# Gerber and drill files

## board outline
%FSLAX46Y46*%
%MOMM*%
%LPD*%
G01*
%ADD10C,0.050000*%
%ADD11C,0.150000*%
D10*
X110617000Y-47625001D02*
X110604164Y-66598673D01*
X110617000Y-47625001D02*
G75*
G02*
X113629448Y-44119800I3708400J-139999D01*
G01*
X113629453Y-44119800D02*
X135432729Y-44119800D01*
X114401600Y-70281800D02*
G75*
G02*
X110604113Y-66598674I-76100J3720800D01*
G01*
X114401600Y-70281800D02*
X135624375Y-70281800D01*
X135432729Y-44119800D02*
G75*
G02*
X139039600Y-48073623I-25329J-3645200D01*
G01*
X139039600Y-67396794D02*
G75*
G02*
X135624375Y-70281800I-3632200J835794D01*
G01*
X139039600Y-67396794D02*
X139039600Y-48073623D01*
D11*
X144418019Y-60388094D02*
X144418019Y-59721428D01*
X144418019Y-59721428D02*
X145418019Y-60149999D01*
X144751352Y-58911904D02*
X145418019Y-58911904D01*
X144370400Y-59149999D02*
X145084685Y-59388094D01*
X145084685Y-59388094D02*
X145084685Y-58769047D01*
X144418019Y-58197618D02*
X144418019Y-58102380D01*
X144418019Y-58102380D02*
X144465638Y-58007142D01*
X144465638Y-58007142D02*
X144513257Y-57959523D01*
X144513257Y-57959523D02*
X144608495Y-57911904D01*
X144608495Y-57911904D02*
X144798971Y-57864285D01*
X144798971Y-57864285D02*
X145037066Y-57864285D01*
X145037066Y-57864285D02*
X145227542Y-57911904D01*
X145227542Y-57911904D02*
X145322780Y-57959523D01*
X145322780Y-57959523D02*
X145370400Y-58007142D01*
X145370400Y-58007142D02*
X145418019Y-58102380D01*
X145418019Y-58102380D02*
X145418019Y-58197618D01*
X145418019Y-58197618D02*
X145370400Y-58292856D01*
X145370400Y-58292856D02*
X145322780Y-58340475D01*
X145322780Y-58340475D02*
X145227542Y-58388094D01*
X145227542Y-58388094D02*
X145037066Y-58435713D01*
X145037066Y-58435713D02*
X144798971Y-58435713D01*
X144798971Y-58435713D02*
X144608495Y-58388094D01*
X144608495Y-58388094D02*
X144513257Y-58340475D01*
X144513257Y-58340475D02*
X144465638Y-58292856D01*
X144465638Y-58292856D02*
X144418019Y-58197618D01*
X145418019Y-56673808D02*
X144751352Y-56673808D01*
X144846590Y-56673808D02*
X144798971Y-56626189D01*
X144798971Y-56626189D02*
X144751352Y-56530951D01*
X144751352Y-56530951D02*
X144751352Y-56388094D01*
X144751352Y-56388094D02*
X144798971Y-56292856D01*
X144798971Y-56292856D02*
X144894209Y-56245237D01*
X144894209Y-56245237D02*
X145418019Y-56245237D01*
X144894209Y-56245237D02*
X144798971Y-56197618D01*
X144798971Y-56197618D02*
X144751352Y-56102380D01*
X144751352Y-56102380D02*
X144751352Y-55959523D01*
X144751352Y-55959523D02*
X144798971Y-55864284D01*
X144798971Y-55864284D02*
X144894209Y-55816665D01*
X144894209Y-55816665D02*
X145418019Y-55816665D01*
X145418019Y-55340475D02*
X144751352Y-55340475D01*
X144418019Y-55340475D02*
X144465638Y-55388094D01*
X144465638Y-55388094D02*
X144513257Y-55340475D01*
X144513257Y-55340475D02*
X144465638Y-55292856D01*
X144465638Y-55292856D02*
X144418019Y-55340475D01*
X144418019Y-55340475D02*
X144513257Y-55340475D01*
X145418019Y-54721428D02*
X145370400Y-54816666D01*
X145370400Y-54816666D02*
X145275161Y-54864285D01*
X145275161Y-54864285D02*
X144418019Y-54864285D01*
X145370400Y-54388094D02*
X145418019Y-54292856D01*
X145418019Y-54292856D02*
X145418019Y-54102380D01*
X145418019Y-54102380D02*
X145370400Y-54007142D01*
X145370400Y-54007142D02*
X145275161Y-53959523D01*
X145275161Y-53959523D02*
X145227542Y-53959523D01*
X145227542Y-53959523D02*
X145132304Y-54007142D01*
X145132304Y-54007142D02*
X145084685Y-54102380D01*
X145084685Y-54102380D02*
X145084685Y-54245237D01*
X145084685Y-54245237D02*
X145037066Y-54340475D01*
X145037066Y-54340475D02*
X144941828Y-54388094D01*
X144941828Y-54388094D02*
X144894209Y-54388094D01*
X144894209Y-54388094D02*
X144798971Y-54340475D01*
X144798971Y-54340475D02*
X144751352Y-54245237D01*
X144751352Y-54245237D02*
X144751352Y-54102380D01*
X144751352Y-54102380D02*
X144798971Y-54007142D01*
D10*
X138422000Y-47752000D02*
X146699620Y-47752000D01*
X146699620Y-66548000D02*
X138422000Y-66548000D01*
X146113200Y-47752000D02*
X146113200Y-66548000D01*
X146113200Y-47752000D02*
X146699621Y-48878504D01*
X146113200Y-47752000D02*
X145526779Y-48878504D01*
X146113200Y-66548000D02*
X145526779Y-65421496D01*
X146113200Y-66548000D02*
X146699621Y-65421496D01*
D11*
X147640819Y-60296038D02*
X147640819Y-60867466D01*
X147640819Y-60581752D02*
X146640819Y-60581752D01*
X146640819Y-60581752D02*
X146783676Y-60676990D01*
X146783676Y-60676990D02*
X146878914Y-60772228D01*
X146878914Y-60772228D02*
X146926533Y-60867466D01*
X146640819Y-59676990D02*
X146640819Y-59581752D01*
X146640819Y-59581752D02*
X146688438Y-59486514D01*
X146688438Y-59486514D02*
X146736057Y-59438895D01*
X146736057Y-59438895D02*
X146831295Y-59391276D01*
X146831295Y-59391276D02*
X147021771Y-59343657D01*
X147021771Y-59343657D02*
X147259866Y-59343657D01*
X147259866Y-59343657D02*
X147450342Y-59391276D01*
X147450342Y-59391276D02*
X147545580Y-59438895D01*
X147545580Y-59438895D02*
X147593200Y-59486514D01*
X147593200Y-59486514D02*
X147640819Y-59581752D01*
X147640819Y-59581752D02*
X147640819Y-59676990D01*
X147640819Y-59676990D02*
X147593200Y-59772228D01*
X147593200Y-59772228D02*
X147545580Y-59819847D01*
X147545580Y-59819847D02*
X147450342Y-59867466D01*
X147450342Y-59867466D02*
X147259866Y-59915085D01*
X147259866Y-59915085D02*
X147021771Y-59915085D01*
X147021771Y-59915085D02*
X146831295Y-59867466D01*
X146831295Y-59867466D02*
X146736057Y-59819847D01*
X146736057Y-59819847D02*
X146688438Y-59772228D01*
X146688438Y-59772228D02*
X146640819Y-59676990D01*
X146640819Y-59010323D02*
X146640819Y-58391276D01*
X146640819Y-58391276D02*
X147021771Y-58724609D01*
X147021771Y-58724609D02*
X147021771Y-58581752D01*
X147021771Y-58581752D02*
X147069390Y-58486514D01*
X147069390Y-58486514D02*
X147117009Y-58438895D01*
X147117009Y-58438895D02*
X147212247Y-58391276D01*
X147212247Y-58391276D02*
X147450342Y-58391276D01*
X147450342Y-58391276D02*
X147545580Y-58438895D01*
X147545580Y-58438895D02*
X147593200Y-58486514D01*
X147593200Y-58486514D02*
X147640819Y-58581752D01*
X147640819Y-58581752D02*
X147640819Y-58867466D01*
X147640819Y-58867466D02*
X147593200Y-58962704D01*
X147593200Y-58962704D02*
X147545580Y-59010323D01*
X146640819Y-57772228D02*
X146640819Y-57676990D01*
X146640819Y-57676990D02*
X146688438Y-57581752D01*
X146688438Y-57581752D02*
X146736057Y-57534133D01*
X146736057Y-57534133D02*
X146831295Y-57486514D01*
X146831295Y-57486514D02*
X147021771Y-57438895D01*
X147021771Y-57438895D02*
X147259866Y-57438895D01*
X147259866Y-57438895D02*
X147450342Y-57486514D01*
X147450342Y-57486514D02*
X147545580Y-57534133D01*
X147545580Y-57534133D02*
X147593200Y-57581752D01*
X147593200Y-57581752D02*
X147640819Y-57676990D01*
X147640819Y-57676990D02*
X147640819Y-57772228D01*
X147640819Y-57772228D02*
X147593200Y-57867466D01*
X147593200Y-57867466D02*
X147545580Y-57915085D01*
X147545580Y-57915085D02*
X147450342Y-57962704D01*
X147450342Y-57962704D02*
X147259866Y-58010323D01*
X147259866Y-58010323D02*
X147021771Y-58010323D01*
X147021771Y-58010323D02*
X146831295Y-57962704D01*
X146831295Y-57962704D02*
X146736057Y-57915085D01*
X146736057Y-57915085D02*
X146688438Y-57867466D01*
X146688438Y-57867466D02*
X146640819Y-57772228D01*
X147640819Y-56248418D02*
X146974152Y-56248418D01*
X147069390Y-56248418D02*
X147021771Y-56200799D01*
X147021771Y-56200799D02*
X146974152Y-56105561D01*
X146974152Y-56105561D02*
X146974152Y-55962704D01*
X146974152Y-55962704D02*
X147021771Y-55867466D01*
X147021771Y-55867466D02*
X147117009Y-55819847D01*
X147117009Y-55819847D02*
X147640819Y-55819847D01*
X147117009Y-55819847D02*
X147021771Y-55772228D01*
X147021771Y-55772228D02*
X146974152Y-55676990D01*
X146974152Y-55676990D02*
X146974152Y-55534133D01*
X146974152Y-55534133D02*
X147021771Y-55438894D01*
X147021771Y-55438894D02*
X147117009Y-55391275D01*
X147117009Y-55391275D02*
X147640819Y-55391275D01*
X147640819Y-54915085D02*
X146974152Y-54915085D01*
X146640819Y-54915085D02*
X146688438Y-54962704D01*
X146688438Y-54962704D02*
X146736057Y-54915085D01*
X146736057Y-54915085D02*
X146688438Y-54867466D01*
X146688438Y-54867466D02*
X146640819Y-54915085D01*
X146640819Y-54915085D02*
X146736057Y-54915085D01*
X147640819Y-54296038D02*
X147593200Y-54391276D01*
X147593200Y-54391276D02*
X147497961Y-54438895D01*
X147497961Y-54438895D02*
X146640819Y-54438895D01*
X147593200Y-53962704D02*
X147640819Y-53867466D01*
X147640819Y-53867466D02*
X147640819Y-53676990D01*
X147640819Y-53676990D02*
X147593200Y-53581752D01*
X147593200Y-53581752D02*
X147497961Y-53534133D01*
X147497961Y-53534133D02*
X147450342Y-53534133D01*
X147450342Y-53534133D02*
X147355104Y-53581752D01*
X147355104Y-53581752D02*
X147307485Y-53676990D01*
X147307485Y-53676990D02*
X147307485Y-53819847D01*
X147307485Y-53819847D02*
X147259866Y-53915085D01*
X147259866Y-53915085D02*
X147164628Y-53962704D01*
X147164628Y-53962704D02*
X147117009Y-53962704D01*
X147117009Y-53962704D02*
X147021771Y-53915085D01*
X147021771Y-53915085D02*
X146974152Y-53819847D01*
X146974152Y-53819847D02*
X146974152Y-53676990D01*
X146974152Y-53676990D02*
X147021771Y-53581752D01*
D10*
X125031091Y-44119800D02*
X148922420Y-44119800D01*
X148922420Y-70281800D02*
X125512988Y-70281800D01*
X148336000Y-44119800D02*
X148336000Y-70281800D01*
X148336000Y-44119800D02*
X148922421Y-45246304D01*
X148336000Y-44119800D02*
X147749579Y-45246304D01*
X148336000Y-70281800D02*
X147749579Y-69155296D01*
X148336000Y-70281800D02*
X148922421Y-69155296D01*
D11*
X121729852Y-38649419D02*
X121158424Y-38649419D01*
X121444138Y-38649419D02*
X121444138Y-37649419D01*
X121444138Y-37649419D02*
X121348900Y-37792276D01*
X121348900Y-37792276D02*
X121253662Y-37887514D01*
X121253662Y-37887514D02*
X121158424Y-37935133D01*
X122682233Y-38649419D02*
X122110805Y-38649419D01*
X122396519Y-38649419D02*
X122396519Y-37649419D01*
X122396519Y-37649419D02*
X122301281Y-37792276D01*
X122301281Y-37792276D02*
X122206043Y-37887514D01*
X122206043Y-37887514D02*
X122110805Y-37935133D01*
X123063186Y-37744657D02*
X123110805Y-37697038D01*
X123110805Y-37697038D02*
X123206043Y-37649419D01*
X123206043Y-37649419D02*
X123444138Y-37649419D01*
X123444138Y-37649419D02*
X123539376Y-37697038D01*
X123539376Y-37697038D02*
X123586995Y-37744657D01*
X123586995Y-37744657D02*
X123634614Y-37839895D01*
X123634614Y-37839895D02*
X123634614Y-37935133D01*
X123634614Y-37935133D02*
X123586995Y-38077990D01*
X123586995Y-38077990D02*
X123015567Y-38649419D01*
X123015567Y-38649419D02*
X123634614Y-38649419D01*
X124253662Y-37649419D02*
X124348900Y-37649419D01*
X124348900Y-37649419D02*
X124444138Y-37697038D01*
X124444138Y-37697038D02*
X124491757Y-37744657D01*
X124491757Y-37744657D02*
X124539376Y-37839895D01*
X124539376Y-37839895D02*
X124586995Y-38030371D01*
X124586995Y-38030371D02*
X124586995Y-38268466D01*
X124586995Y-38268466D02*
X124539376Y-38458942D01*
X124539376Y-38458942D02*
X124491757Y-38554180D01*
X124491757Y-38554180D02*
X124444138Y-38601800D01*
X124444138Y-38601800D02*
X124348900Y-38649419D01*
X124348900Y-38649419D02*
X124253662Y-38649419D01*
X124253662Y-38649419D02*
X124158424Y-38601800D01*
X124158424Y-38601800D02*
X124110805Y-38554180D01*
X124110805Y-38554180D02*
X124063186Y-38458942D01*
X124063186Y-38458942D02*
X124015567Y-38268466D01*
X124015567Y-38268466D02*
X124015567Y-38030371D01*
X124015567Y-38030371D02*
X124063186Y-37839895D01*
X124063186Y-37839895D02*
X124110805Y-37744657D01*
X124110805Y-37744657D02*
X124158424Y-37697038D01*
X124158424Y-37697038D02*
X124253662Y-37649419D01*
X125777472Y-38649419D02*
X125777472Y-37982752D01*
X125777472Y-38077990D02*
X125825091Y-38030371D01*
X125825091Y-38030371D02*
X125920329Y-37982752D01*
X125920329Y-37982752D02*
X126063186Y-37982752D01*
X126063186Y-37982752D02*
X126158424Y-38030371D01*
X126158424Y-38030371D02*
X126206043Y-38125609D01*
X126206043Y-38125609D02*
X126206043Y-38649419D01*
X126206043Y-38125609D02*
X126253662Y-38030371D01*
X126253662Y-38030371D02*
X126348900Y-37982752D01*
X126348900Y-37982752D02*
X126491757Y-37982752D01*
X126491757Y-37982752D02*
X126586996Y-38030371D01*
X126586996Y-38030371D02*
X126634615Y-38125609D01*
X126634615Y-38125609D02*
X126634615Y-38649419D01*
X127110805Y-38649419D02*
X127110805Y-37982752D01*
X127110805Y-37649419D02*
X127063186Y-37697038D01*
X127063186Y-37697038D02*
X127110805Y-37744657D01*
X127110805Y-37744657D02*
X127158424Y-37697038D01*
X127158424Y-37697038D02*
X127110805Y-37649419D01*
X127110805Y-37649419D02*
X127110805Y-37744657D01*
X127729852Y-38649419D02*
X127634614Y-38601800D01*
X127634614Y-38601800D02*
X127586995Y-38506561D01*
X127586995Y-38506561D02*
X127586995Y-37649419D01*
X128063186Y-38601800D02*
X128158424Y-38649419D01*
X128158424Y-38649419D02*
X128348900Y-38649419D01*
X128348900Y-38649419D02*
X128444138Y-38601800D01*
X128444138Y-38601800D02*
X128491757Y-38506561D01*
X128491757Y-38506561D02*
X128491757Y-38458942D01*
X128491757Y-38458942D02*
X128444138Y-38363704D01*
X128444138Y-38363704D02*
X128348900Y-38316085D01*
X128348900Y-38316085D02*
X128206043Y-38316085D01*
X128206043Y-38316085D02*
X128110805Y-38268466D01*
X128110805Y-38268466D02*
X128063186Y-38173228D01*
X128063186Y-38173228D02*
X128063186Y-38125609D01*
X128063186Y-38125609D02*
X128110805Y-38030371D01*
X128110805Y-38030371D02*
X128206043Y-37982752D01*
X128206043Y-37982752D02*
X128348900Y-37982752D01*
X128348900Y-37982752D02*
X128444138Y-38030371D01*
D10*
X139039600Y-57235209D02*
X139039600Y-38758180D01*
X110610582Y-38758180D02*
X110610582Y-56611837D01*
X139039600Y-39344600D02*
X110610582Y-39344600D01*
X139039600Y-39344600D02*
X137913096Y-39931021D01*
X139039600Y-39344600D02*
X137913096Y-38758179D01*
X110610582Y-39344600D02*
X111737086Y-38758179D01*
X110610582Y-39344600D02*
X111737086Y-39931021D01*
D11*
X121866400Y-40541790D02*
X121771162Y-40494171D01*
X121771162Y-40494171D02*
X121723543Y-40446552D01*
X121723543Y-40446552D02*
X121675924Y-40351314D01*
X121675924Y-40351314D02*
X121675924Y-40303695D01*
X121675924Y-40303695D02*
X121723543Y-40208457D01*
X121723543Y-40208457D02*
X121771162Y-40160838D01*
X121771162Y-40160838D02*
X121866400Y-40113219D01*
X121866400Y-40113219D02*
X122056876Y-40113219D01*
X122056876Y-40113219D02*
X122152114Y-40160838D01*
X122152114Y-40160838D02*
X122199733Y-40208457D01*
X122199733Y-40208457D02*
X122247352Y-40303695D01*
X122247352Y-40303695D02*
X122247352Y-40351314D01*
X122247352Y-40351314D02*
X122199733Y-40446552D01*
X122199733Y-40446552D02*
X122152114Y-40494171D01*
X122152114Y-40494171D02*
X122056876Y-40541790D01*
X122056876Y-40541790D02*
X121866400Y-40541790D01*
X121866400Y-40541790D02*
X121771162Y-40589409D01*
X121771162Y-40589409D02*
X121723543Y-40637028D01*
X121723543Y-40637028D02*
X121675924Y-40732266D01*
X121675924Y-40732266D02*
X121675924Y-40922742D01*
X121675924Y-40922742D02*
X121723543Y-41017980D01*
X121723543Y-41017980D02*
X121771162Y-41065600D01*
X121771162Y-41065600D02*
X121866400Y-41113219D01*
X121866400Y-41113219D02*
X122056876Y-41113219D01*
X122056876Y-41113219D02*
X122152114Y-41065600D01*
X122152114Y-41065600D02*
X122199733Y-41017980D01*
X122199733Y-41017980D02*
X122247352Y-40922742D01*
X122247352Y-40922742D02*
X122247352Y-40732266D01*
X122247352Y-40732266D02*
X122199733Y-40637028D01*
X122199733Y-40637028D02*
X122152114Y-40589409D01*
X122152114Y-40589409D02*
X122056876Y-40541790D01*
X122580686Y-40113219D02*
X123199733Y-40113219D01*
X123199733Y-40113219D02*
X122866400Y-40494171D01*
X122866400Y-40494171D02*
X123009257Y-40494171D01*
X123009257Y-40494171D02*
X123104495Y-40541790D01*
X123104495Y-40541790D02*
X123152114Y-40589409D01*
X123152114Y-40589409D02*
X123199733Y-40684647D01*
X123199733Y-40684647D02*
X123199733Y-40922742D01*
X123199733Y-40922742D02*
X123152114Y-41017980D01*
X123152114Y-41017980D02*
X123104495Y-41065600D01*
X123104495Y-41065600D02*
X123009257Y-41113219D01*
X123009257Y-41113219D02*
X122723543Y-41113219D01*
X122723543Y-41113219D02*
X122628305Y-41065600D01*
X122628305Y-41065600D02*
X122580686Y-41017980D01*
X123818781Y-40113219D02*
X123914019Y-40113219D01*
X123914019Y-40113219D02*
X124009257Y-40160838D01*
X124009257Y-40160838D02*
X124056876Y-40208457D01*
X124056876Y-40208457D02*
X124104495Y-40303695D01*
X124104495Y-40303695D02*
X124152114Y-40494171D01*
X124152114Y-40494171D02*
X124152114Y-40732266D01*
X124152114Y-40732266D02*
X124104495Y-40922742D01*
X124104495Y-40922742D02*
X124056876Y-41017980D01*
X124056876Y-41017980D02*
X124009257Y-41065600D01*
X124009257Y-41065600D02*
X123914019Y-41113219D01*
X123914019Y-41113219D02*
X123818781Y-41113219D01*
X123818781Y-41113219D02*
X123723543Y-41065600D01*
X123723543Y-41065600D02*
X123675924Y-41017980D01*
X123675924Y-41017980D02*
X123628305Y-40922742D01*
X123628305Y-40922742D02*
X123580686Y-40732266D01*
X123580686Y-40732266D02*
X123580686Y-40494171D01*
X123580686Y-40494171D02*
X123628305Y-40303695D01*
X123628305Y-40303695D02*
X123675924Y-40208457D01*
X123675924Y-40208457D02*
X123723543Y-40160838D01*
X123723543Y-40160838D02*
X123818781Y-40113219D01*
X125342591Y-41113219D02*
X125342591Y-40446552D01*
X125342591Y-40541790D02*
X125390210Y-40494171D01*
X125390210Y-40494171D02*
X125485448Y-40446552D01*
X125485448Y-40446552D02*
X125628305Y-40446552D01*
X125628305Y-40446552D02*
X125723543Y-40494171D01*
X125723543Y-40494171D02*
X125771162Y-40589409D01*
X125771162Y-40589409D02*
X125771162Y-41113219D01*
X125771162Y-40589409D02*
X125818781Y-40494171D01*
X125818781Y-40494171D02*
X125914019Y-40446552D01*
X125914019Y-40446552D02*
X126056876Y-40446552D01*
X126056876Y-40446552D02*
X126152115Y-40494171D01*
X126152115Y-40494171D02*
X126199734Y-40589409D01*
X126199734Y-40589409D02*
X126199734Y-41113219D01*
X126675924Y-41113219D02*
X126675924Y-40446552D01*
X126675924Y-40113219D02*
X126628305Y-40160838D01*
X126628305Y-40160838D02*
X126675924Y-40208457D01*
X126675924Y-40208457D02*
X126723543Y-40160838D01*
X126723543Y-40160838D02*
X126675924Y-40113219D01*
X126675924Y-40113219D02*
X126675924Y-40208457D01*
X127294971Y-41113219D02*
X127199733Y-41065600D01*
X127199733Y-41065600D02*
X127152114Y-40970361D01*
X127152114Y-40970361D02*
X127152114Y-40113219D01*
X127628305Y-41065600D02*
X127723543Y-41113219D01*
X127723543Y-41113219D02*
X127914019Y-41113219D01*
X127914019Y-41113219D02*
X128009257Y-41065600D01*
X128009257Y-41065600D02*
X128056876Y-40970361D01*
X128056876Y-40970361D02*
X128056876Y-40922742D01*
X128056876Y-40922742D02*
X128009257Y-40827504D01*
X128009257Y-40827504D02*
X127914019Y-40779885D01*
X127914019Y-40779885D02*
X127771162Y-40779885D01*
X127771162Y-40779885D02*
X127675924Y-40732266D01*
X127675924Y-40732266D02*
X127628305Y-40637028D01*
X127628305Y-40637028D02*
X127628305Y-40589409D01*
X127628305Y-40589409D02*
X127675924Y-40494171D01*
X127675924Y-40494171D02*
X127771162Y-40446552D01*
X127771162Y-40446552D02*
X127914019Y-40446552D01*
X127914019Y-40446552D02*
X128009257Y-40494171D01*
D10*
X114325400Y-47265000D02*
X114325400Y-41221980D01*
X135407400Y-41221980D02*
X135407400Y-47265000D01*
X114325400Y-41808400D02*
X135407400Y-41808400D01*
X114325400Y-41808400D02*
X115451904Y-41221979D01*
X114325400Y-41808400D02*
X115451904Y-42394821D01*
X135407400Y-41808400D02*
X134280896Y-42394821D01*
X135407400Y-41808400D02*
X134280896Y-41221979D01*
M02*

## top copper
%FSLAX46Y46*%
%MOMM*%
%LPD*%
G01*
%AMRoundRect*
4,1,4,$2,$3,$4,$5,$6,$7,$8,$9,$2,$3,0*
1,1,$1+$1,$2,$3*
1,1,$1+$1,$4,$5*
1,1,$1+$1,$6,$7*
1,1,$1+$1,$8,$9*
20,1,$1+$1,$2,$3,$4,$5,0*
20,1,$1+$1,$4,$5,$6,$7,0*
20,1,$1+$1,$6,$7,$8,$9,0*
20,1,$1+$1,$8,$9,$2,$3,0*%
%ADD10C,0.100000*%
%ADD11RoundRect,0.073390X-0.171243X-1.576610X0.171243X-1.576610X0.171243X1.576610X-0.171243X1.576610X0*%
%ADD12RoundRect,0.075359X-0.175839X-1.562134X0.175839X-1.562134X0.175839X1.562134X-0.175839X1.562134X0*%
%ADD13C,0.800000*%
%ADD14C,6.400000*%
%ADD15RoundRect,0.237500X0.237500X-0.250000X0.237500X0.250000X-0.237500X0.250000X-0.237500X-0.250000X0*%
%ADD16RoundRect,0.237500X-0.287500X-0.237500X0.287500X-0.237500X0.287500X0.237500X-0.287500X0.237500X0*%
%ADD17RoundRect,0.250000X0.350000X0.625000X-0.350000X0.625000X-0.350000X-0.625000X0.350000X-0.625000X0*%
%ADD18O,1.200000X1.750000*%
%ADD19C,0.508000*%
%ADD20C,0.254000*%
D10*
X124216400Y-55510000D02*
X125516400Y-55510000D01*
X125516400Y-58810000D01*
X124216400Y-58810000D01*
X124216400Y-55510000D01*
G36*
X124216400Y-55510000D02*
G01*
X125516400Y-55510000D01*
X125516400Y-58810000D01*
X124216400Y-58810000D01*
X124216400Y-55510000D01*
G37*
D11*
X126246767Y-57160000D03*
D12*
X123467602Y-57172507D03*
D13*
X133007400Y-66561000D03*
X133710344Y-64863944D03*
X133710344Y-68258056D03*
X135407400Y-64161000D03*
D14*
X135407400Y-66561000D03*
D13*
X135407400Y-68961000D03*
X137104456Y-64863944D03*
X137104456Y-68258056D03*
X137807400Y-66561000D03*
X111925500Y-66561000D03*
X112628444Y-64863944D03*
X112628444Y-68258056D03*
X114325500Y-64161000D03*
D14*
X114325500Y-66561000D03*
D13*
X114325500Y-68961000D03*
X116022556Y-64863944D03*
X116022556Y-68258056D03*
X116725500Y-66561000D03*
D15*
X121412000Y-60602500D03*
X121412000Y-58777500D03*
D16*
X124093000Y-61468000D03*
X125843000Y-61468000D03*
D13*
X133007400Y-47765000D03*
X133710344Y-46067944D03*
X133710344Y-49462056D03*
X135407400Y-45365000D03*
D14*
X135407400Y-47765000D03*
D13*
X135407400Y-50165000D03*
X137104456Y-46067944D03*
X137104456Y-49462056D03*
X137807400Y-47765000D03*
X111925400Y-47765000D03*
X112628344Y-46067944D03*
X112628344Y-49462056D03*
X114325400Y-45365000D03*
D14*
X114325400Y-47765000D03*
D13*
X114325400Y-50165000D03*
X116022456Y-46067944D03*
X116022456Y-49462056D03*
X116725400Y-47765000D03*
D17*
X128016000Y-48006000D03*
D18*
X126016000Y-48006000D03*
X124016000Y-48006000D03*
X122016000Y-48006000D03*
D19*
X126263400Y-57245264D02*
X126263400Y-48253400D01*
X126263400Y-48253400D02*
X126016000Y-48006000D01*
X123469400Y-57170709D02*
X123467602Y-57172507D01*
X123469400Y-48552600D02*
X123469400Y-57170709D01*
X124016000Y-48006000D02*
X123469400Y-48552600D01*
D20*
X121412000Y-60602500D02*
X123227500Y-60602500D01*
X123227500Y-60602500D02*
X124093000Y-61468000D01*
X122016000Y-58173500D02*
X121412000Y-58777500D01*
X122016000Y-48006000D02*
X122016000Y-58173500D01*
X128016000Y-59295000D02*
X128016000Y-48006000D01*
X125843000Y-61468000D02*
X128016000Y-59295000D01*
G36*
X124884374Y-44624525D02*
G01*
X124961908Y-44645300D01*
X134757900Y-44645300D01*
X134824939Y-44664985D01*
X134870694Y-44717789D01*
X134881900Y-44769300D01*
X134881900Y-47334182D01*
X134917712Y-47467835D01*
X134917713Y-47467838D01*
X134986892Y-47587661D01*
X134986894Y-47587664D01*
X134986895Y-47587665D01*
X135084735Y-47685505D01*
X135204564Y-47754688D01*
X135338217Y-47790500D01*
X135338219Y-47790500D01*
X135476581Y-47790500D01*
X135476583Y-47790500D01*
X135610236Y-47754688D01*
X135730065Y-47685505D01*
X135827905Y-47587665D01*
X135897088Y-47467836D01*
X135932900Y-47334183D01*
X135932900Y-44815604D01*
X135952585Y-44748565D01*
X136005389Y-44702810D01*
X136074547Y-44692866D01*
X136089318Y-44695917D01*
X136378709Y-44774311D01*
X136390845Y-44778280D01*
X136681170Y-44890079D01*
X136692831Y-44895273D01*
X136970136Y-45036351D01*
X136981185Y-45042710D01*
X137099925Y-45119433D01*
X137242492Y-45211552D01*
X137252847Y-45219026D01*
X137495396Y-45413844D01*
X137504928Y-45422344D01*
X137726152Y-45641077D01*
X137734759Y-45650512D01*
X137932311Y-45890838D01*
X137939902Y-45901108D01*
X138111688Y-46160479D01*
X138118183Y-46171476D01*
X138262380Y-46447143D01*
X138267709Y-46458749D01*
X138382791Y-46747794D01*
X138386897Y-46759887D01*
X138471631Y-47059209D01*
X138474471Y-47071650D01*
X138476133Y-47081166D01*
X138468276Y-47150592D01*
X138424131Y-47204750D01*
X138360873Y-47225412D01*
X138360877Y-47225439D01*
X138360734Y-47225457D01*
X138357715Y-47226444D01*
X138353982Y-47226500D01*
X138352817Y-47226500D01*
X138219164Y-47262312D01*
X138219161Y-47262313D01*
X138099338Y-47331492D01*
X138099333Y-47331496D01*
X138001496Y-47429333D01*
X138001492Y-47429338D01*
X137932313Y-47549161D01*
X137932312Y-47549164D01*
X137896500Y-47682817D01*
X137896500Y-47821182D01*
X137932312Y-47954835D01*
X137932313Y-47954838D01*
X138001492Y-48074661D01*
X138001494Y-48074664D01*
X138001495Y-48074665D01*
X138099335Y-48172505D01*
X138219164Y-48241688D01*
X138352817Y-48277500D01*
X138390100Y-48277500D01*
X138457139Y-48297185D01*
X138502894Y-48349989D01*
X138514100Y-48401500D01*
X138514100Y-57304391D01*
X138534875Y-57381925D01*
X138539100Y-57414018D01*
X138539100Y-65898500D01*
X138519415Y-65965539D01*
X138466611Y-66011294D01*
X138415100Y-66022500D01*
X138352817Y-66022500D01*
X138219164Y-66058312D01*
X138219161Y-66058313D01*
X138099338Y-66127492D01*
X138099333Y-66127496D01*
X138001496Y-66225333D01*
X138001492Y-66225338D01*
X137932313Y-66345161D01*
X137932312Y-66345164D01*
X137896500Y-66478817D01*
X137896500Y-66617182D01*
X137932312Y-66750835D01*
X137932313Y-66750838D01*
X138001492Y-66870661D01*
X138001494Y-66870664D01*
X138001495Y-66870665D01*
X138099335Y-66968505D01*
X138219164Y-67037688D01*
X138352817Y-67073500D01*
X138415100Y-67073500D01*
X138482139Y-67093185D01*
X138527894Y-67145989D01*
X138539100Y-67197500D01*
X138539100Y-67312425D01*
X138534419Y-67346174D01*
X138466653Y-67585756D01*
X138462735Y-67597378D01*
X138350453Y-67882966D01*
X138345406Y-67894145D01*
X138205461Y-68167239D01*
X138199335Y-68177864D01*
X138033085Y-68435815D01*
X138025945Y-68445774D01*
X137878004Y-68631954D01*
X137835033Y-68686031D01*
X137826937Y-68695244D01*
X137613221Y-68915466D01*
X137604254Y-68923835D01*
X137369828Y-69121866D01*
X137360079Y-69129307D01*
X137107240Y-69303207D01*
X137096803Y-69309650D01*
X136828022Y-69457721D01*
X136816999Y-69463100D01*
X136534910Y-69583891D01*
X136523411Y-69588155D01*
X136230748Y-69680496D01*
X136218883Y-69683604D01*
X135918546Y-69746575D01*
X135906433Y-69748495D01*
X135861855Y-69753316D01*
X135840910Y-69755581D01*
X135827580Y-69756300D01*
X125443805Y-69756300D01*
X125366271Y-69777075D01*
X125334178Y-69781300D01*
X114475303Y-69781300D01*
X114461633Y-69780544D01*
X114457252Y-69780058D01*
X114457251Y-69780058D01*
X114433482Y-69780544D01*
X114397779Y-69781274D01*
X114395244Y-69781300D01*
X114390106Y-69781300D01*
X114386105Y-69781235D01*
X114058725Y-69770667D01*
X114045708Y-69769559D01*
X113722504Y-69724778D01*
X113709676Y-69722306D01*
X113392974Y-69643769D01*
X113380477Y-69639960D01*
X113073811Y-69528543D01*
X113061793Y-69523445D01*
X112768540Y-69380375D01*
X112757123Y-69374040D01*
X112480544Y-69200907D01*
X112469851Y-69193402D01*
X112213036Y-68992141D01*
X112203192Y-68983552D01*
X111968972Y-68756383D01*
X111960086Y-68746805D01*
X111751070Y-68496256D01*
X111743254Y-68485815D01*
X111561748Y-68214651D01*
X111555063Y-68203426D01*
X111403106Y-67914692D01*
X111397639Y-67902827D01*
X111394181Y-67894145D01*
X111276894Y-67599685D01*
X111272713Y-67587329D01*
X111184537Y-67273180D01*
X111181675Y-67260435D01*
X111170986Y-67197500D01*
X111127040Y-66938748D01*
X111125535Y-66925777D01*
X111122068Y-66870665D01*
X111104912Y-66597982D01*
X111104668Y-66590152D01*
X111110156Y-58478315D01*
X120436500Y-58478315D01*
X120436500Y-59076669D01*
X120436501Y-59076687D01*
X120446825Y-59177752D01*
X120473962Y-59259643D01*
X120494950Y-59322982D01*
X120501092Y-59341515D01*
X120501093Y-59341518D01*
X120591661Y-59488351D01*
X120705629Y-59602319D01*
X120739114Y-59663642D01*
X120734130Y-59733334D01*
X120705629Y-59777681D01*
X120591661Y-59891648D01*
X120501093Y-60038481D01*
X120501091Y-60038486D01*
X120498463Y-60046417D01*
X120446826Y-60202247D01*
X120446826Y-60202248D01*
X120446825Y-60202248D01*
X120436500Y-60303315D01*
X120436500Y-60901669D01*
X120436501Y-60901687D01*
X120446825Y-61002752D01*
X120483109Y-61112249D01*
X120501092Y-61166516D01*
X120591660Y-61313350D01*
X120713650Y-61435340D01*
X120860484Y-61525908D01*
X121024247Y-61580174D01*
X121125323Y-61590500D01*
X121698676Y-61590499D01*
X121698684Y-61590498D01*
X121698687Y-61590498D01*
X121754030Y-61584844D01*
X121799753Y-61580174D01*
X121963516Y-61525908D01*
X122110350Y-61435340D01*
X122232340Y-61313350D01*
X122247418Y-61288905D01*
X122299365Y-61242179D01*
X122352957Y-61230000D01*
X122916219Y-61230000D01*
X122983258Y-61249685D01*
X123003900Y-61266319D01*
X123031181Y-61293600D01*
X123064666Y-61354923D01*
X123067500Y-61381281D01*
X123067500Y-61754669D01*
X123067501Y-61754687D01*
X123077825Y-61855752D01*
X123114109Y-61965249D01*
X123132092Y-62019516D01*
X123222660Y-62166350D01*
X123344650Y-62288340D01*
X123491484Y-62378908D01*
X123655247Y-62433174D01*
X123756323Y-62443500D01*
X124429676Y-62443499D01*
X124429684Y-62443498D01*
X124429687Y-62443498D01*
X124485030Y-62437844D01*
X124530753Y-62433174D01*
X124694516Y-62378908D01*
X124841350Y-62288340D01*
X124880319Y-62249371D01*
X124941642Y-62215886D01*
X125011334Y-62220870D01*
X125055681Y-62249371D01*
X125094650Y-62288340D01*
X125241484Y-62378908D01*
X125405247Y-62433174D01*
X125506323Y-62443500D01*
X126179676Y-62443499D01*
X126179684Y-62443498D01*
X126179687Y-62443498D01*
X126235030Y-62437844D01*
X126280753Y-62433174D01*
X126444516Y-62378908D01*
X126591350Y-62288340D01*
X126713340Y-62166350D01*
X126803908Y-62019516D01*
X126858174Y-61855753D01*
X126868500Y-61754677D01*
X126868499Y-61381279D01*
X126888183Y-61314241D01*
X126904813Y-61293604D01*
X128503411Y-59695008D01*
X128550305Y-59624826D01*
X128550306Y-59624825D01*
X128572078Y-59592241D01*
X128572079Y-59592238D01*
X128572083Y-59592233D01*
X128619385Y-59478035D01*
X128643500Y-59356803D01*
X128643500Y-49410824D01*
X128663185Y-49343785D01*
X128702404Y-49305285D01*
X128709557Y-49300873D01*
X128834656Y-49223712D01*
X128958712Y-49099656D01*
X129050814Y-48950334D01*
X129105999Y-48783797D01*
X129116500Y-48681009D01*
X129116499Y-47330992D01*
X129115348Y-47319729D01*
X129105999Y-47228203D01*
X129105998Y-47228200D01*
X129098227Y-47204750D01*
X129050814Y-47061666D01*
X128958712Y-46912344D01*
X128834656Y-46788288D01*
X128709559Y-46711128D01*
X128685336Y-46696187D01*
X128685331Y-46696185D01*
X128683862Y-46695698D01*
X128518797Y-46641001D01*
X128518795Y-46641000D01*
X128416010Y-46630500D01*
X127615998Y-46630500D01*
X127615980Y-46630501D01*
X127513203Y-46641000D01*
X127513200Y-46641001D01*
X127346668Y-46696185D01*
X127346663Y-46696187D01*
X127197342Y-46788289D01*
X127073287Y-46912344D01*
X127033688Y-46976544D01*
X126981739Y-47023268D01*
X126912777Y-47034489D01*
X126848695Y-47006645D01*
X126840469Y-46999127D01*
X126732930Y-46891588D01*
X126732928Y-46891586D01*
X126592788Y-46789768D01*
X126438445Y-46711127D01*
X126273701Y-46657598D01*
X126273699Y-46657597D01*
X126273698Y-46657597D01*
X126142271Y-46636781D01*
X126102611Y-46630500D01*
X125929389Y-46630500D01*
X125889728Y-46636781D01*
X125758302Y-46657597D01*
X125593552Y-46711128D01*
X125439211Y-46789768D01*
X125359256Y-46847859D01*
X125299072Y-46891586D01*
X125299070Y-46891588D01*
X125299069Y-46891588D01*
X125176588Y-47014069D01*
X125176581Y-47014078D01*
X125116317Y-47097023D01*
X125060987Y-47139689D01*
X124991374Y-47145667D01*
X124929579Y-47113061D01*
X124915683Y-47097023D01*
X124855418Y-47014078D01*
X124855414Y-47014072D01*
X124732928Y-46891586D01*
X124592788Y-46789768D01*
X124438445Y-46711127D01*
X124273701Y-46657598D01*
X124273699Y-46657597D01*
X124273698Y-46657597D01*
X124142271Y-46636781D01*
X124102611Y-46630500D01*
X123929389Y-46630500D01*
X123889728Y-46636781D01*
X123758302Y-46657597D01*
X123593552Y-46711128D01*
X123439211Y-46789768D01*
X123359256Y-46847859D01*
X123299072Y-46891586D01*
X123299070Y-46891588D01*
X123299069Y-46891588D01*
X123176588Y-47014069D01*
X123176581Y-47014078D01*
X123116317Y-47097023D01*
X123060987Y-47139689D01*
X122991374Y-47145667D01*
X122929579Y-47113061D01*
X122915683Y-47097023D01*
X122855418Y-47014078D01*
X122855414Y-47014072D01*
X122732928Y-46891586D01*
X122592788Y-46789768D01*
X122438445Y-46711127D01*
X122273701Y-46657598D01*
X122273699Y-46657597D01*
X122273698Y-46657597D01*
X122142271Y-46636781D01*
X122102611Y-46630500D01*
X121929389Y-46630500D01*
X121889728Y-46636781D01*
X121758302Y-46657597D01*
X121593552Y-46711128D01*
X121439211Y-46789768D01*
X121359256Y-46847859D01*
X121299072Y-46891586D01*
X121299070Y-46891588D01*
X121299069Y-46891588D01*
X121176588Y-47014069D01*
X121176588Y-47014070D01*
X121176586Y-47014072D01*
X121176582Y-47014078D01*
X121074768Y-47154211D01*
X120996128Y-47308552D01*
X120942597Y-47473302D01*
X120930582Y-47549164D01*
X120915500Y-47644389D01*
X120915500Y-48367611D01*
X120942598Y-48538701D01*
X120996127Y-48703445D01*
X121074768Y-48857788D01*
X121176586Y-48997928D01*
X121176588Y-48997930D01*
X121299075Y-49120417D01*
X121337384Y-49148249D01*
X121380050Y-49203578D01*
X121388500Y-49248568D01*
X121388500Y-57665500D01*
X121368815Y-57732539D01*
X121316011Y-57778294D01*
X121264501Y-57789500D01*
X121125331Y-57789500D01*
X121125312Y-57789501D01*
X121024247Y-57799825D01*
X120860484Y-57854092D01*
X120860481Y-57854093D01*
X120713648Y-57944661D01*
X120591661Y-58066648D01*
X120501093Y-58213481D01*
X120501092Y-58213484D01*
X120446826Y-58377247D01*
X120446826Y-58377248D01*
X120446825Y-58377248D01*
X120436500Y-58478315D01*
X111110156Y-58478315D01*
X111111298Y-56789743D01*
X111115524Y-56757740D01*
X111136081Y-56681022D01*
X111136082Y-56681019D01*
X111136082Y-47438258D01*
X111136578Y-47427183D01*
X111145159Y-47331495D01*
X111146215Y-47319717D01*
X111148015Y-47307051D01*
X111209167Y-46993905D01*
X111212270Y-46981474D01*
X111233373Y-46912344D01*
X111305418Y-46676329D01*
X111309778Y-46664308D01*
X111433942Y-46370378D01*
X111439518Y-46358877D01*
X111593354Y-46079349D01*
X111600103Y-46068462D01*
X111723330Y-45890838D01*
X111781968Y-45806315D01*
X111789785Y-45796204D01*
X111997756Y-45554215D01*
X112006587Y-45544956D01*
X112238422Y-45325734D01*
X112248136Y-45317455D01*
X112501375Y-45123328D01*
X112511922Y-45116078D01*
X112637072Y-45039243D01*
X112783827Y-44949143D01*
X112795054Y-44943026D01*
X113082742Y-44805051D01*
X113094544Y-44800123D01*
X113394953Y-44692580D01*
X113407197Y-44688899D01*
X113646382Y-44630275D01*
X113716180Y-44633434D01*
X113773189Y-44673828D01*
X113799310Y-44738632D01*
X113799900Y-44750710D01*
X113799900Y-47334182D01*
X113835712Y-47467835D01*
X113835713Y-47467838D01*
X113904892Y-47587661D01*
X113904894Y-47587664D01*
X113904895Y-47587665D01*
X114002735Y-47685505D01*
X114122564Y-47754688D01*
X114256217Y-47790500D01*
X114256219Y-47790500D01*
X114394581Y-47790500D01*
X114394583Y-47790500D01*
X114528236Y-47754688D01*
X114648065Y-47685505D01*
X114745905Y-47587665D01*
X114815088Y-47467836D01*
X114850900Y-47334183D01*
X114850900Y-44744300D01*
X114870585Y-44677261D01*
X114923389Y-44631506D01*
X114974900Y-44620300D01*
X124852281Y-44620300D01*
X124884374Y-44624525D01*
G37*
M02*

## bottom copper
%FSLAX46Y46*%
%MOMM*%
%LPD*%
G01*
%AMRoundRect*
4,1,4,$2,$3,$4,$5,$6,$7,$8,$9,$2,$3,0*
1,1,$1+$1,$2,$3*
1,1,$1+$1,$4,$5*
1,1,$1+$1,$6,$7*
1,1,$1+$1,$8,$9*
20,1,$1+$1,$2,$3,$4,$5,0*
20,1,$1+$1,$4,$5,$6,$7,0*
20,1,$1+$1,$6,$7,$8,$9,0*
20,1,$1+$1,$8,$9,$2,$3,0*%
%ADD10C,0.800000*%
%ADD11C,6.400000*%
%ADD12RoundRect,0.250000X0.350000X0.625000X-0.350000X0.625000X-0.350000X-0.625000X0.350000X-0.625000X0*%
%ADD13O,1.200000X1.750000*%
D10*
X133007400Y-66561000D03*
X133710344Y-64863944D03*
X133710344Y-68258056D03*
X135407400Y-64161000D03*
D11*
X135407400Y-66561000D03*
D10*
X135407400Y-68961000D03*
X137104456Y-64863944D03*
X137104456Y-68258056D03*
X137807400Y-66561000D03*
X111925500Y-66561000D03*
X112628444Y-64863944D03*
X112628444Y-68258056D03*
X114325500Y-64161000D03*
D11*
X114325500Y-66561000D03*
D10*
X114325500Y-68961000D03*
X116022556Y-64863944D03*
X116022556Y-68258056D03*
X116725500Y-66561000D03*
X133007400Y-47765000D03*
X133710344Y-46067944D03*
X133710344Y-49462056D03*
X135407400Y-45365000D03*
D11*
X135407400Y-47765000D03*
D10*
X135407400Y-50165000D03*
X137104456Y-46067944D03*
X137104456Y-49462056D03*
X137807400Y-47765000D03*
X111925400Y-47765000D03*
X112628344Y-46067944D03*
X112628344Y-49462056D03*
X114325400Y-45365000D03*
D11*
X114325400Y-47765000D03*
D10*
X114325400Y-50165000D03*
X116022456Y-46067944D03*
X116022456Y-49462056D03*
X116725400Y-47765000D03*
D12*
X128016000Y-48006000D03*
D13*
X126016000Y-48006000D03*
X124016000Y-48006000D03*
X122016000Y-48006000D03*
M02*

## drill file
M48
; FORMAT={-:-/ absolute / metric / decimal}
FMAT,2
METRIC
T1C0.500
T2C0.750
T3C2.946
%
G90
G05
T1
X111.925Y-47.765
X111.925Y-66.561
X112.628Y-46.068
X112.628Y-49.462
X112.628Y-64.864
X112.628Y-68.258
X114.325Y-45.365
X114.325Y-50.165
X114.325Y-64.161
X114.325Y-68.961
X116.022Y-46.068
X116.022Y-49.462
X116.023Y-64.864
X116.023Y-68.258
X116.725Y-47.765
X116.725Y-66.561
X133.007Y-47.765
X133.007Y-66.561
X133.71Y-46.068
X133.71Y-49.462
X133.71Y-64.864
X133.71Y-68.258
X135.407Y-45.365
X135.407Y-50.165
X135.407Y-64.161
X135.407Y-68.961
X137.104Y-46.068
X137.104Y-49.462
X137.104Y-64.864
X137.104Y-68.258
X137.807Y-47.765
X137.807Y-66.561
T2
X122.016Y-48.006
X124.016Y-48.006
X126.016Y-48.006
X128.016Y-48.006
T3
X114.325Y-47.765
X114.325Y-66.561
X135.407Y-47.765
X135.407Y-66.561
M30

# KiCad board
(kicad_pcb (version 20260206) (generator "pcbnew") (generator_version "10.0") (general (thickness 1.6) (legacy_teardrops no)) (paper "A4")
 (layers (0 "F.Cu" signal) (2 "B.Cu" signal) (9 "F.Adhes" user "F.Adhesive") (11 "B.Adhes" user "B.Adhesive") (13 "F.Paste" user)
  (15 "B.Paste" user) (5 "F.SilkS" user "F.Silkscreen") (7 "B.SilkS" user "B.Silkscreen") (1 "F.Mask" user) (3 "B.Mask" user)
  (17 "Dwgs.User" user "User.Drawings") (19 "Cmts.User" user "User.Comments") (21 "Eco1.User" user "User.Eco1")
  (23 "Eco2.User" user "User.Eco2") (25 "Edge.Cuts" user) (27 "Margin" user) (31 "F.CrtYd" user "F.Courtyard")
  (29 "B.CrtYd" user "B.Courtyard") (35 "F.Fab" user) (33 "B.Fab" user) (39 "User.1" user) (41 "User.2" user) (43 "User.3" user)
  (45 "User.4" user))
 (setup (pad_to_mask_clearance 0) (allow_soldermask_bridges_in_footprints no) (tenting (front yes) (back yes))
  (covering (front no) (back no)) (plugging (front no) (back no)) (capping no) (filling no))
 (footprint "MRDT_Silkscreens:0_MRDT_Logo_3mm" (layer "F.Cu") (at 131.8006 60.7568 -90)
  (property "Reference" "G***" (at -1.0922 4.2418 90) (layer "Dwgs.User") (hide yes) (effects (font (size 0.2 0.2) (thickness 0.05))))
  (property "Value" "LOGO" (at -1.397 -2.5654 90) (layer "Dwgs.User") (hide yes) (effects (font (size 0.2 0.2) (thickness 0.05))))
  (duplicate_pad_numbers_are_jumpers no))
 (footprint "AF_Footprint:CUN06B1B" (layer "F.Cu") (at 124.8664 57.163)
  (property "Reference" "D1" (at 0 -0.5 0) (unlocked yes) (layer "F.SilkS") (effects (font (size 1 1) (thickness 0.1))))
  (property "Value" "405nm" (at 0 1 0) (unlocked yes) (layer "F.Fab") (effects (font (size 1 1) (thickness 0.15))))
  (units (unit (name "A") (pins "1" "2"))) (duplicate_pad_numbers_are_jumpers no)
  (fp_rect (start -0.65 -1.653) (end 0.65 1.647) (stroke (width 0.1) (type solid)) (fill yes) (layer "F.Cu"))
  (pad "1" smd roundrect (at 1.380367 -0.003) (size 0.489266 3.3) (layers "F.Cu" "F.Mask" "F.Paste") (roundrect_rratio 0.15)
   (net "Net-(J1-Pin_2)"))
  (pad "2" smd roundrect (at -1.398798 0.009507) (size 0.502396 3.274986) (layers "F.Cu" "F.Mask" "F.Paste") (roundrect_rratio 0.15)
   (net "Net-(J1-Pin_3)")))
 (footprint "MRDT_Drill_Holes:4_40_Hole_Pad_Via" (layer "F.Cu") (at 135.4074 66.561)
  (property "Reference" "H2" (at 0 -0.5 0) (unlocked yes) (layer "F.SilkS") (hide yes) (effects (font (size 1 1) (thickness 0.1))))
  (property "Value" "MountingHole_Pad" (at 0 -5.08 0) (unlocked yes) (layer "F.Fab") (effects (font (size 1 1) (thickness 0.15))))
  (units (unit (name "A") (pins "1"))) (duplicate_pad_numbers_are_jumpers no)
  (pad "1" thru_hole circle (at -2.4 0) (size 0.8 0.8) (drill 0.5) (layers "*.Cu" "*.Mask") (remove_unused_layers no) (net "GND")
   (zone_connect 2))
  (pad "1" thru_hole circle (at -1.697056 -1.697056) (size 0.8 0.8) (drill 0.5) (layers "*.Cu" "*.Mask") (remove_unused_layers no)
   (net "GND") (zone_connect 2))
  (pad "1" thru_hole circle (at -1.697056 1.697056) (size 0.8 0.8) (drill 0.5) (layers "*.Cu" "*.Mask") (remove_unused_layers no)
   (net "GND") (zone_connect 2))
  (pad "1" thru_hole circle (at 0 -2.4) (size 0.8 0.8) (drill 0.5) (layers "*.Cu" "*.Mask") (remove_unused_layers no) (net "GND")
   (zone_connect 2))
  (pad "1" thru_hole circle (at 0 0) (size 6.4 6.4) (drill 2.9464) (layers "*.Cu" "*.Mask") (remove_unused_layers no) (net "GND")
   (zone_connect 2))
  (pad "1" thru_hole circle (at 0 2.4) (size 0.8 0.8) (drill 0.5) (layers "*.Cu" "*.Mask") (remove_unused_layers no) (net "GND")
   (zone_connect 2))
  (pad "1" thru_hole circle (at 1.697056 -1.697056) (size 0.8 0.8) (drill 0.5) (layers "*.Cu" "*.Mask") (remove_unused_layers no)
   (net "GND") (zone_connect 2))
  (pad "1" thru_hole circle (at 1.697056 1.697056) (size 0.8 0.8) (drill 0.5) (layers "*.Cu" "*.Mask") (remove_unused_layers no) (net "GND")
   (zone_connect 2))
  (pad "1" thru_hole circle (at 2.4 0) (size 0.8 0.8) (drill 0.5) (layers "*.Cu" "*.Mask") (remove_unused_layers no) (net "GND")
   (zone_connect 2)))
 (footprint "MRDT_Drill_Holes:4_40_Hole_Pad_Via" (layer "F.Cu") (at 114.3255 66.561)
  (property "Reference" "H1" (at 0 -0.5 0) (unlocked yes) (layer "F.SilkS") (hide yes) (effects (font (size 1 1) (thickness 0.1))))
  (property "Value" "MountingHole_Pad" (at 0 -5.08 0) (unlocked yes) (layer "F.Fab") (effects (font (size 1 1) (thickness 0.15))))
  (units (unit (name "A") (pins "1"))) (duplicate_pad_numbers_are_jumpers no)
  (pad "1" thru_hole circle (at -2.4 0) (size 0.8 0.8) (drill 0.5) (layers "*.Cu" "*.Mask") (remove_unused_layers no) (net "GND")
   (zone_connect 2))
  (pad "1" thru_hole circle (at -1.697056 -1.697056) (size 0.8 0.8) (drill 0.5) (layers "*.Cu" "*.Mask") (remove_unused_layers no)
   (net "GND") (zone_connect 2))
  (pad "1" thru_hole circle (at -1.697056 1.697056) (size 0.8 0.8) (drill 0.5) (layers "*.Cu" "*.Mask") (remove_unused_layers no)
   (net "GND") (zone_connect 2))
  (pad "1" thru_hole circle (at 0 -2.4) (size 0.8 0.8) (drill 0.5) (layers "*.Cu" "*.Mask") (remove_unused_layers no) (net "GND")
   (zone_connect 2))
  (pad "1" thru_hole circle (at 0 0) (size 6.4 6.4) (drill 2.9464) (layers "*.Cu" "*.Mask") (remove_unused_layers no) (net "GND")
   (zone_connect 2))
  (pad "1" thru_hole circle (at 0 2.4) (size 0.8 0.8) (drill 0.5) (layers "*.Cu" "*.Mask") (remove_unused_layers no) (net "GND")
   (zone_connect 2))
  (pad "1" thru_hole circle (at 1.697056 -1.697056) (size 0.8 0.8) (drill 0.5) (layers "*.Cu" "*.Mask") (remove_unused_layers no)
   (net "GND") (zone_connect 2))
  (pad "1" thru_hole circle (at 1.697056 1.697056) (size 0.8 0.8) (drill 0.5) (layers "*.Cu" "*.Mask") (remove_unused_layers no) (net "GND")
   (zone_connect 2))
  (pad "1" thru_hole circle (at 2.4 0) (size 0.8 0.8) (drill 0.5) (layers "*.Cu" "*.Mask") (remove_unused_layers no) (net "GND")
   (zone_connect 2)))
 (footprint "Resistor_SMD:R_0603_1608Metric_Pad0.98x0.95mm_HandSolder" (layer "F.Cu") (at 121.412 59.69 90)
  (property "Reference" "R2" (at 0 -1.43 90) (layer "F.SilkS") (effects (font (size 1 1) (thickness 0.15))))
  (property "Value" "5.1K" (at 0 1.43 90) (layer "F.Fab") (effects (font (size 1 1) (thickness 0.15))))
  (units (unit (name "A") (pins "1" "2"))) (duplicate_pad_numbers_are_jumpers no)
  (pad "1" smd roundrect (at -0.9125 0 90) (size 0.975 0.95) (layers "F.Cu" "F.Mask" "F.Paste") (roundrect_rratio 0.25) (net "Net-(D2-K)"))
  (pad "2" smd roundrect (at 0.9125 0 90) (size 0.975 0.95) (layers "F.Cu" "F.Mask" "F.Paste") (roundrect_rratio 0.25)
   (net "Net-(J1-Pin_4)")))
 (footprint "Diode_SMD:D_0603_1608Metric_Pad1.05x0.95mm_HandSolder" (layer "F.Cu") (at 124.968 61.468)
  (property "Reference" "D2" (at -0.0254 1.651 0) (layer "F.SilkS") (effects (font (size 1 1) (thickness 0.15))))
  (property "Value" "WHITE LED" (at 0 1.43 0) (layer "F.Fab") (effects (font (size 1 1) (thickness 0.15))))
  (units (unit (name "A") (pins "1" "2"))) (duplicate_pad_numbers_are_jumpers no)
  (pad "1" smd roundrect (at -0.875 0) (size 1.05 0.95) (layers "F.Cu" "F.Mask" "F.Paste") (roundrect_rratio 0.25) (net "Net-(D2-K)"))
  (pad "2" smd roundrect (at 0.875 0) (size 1.05 0.95) (layers "F.Cu" "F.Mask" "F.Paste") (roundrect_rratio 0.25) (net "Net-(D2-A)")))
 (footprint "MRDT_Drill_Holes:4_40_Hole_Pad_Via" (layer "F.Cu") (at 135.4074 47.765)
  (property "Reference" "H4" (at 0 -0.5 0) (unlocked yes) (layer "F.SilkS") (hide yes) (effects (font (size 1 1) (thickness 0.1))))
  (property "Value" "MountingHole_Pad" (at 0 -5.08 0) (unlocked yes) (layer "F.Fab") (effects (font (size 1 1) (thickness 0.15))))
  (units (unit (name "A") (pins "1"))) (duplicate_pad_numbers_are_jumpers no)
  (pad "1" thru_hole circle (at -2.4 0) (size 0.8 0.8) (drill 0.5) (layers "*.Cu" "*.Mask") (remove_unused_layers no) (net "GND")
   (zone_connect 2))
  (pad "1" thru_hole circle (at -1.697056 -1.697056) (size 0.8 0.8) (drill 0.5) (layers "*.Cu" "*.Mask") (remove_unused_layers no)
   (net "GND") (zone_connect 2))
  (pad "1" thru_hole circle (at -1.697056 1.697056) (size 0.8 0.8) (drill 0.5) (layers "*.Cu" "*.Mask") (remove_unused_layers no)
   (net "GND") (zone_connect 2))
  (pad "1" thru_hole circle (at 0 -2.4) (size 0.8 0.8) (drill 0.5) (layers "*.Cu" "*.Mask") (remove_unused_layers no) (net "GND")
   (zone_connect 2))
  (pad "1" thru_hole circle (at 0 0) (size 6.4 6.4) (drill 2.9464) (layers "*.Cu" "*.Mask") (remove_unused_layers no) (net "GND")
   (zone_connect 2))
  (pad "1" thru_hole circle (at 0 2.4) (size 0.8 0.8) (drill 0.5) (layers "*.Cu" "*.Mask") (remove_unused_layers no) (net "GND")
   (zone_connect 2))
  (pad "1" thru_hole circle (at 1.697056 -1.697056) (size 0.8 0.8) (drill 0.5) (layers "*.Cu" "*.Mask") (remove_unused_layers no)
   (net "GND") (zone_connect 2))
  (pad "1" thru_hole circle (at 1.697056 1.697056) (size 0.8 0.8) (drill 0.5) (layers "*.Cu" "*.Mask") (remove_unused_layers no) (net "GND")
   (zone_connect 2))
  (pad "1" thru_hole circle (at 2.4 0) (size 0.8 0.8) (drill 0.5) (layers "*.Cu" "*.Mask") (remove_unused_layers no) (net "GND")
   (zone_connect 2)))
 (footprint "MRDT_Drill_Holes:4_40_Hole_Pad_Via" (layer "F.Cu") (at 114.3254 47.765)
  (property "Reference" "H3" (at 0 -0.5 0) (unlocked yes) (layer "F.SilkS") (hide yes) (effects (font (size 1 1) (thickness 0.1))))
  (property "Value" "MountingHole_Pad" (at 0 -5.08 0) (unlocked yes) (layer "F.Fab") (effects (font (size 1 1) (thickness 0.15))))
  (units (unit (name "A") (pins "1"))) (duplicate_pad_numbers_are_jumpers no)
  (pad "1" thru_hole circle (at -2.4 0) (size 0.8 0.8) (drill 0.5) (layers "*.Cu" "*.Mask") (remove_unused_layers no) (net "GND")
   (zone_connect 2))
  (pad "1" thru_hole circle (at -1.697056 -1.697056) (size 0.8 0.8) (drill 0.5) (layers "*.Cu" "*.Mask") (remove_unused_layers no)
   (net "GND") (zone_connect 2))
  (pad "1" thru_hole circle (at -1.697056 1.697056) (size 0.8 0.8) (drill 0.5) (layers "*.Cu" "*.Mask") (remove_unused_layers no)
   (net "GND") (zone_connect 2))
  (pad "1" thru_hole circle (at 0 -2.4) (size 0.8 0.8) (drill 0.5) (layers "*.Cu" "*.Mask") (remove_unused_layers no) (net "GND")
   (zone_connect 2))
  (pad "1" thru_hole circle (at 0 0) (size 6.4 6.4) (drill 2.9464) (layers "*.Cu" "*.Mask") (remove_unused_layers no) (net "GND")
   (zone_connect 2))
  (pad "1" thru_hole circle (at 0 2.4) (size 0.8 0.8) (drill 0.5) (layers "*.Cu" "*.Mask") (remove_unused_layers no) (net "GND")
   (zone_connect 2))
  (pad "1" thru_hole circle (at 1.697056 -1.697056) (size 0.8 0.8) (drill 0.5) (layers "*.Cu" "*.Mask") (remove_unused_layers no)
   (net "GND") (zone_connect 2))
  (pad "1" thru_hole circle (at 1.697056 1.697056) (size 0.8 0.8) (drill 0.5) (layers "*.Cu" "*.Mask") (remove_unused_layers no) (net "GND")
   (zone_connect 2))
  (pad "1" thru_hole circle (at 2.4 0) (size 0.8 0.8) (drill 0.5) (layers "*.Cu" "*.Mask") (remove_unused_layers no) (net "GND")
   (zone_connect 2)))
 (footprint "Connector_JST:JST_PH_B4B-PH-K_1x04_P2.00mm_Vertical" (layer "B.Cu") (at 128.016 48.006 180)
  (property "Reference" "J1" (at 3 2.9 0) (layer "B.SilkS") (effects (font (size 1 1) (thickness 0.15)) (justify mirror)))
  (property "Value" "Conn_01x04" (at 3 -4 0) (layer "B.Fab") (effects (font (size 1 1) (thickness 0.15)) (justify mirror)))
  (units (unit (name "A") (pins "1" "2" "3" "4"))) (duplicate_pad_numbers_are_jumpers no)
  (pad "1" thru_hole roundrect (at 0 0 180) (size 1.2 1.75) (drill 0.75) (layers "*.Cu" "*.Mask") (remove_unused_layers no)
   (roundrect_rratio 0.208333) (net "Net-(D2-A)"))
  (pad "2" thru_hole oval (at 2 0 180) (size 1.2 1.75) (drill 0.75) (layers "*.Cu" "*.Mask") (remove_unused_layers no)
   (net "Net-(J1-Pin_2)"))
  (pad "3" thru_hole oval (at 4 0 180) (size 1.2 1.75) (drill 0.75) (layers "*.Cu" "*.Mask") (remove_unused_layers no)
   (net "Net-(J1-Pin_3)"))
  (pad "4" thru_hole oval (at 6 0 180) (size 1.2 1.75) (drill 0.75) (layers "*.Cu" "*.Mask") (remove_unused_layers no)
   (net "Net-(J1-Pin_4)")))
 (gr_line (start 110.617 47.625001) (end 110.604164 66.598673) (stroke (width 0.05) (type default)) (layer "Edge.Cuts"))
 (gr_arc (start 110.617 47.625001) (mid 111.51094 45.34619) (end 113.629448 44.1198) (stroke (width 0.05) (type solid)) (layer "Edge.Cuts"))
 (gr_line (start 113.629453 44.1198) (end 135.432729 44.1198) (stroke (width 0.05) (type default)) (layer "Edge.Cuts"))
 (gr_arc (start 114.4016 70.2818) (mid 111.734512 69.232453) (end 110.604164 66.598673) (stroke (width 0.05) (type solid))
  (layer "Edge.Cuts"))
 (gr_line (start 114.4016 70.2818) (end 135.624375 70.2818) (stroke (width 0.05) (type default)) (layer "Edge.Cuts"))
 (gr_arc (start 135.432729 44.1198) (mid 138.100457 45.308261) (end 139.0396 48.073623) (stroke (width 0.05) (type solid))
  (layer "Edge.Cuts"))
 (gr_arc (start 139.0396 67.396794) (mid 137.812572 69.408205) (end 135.624375 70.2818) (stroke (width 0.05) (type solid))
  (layer "Edge.Cuts"))
 (gr_line (start 139.0396 67.396794) (end 139.0396 48.073623) (stroke (width 0.05) (type default)) (layer "Edge.Cuts"))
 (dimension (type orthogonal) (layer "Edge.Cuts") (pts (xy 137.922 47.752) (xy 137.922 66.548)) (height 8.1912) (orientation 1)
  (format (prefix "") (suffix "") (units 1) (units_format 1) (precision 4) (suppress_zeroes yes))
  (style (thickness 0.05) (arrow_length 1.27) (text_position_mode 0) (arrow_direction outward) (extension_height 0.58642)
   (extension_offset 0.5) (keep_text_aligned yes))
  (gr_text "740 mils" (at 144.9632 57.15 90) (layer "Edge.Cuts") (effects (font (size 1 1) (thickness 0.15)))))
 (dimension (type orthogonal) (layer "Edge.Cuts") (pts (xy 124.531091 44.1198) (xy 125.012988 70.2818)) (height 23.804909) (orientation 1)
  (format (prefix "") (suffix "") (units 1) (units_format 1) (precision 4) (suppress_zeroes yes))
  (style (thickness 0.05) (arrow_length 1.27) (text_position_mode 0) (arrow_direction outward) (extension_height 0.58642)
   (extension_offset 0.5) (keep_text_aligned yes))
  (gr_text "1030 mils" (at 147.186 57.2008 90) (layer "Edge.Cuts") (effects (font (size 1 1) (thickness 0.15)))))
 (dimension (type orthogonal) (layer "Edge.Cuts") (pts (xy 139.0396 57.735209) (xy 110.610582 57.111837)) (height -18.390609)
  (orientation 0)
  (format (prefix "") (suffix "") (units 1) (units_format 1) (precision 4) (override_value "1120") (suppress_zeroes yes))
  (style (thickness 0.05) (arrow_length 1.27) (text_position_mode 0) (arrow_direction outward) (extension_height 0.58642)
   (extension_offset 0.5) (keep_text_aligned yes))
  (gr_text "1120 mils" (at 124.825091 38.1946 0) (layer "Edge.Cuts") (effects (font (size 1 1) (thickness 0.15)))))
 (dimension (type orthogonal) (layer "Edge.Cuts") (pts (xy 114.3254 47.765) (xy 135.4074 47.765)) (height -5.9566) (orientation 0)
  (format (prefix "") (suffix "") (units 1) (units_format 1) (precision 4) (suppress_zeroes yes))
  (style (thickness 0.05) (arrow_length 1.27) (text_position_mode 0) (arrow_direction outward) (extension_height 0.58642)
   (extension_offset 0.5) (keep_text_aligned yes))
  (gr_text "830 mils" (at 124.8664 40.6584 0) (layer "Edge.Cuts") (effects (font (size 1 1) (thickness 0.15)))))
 (segment (start 126.2634 57.245264) (end 126.2634 48.2534) (width 0.508) (layer "F.Cu") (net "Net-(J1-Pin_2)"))
 (segment (start 126.2634 48.2534) (end 126.016 48.006) (width 0.508) (layer "F.Cu") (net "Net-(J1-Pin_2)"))
 (segment (start 123.4694 57.170709) (end 123.467602 57.172507) (width 0.508) (layer "F.Cu") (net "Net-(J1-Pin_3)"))
 (segment (start 123.4694 48.5526) (end 123.4694 57.170709) (width 0.508) (layer "F.Cu") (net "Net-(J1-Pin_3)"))
 (segment (start 124.016 48.006) (end 123.4694 48.5526) (width 0.508) (layer "F.Cu") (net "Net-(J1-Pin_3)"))
 (segment (start 121.412 60.6025) (end 123.2275 60.6025) (width 0.254) (layer "F.Cu") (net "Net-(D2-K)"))
 (segment (start 123.2275 60.6025) (end 124.093 61.468) (width 0.254) (layer "F.Cu") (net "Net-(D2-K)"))
 (segment (start 122.016 58.1735) (end 121.412 58.7775) (width 0.254) (layer "F.Cu") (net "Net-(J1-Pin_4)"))
 (segment (start 122.016 48.006) (end 122.016 58.1735) (width 0.254) (layer "F.Cu") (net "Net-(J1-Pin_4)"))
 (segment (start 128.016 59.295) (end 128.016 48.006) (width 0.254) (layer "F.Cu") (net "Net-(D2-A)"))
 (segment (start 125.843 61.468) (end 128.016 59.295) (width 0.254) (layer "F.Cu") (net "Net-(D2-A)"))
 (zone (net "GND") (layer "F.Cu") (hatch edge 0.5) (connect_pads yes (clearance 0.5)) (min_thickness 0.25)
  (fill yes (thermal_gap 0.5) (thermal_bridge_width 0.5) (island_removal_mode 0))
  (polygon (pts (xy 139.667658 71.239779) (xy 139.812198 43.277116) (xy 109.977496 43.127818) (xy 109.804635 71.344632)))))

